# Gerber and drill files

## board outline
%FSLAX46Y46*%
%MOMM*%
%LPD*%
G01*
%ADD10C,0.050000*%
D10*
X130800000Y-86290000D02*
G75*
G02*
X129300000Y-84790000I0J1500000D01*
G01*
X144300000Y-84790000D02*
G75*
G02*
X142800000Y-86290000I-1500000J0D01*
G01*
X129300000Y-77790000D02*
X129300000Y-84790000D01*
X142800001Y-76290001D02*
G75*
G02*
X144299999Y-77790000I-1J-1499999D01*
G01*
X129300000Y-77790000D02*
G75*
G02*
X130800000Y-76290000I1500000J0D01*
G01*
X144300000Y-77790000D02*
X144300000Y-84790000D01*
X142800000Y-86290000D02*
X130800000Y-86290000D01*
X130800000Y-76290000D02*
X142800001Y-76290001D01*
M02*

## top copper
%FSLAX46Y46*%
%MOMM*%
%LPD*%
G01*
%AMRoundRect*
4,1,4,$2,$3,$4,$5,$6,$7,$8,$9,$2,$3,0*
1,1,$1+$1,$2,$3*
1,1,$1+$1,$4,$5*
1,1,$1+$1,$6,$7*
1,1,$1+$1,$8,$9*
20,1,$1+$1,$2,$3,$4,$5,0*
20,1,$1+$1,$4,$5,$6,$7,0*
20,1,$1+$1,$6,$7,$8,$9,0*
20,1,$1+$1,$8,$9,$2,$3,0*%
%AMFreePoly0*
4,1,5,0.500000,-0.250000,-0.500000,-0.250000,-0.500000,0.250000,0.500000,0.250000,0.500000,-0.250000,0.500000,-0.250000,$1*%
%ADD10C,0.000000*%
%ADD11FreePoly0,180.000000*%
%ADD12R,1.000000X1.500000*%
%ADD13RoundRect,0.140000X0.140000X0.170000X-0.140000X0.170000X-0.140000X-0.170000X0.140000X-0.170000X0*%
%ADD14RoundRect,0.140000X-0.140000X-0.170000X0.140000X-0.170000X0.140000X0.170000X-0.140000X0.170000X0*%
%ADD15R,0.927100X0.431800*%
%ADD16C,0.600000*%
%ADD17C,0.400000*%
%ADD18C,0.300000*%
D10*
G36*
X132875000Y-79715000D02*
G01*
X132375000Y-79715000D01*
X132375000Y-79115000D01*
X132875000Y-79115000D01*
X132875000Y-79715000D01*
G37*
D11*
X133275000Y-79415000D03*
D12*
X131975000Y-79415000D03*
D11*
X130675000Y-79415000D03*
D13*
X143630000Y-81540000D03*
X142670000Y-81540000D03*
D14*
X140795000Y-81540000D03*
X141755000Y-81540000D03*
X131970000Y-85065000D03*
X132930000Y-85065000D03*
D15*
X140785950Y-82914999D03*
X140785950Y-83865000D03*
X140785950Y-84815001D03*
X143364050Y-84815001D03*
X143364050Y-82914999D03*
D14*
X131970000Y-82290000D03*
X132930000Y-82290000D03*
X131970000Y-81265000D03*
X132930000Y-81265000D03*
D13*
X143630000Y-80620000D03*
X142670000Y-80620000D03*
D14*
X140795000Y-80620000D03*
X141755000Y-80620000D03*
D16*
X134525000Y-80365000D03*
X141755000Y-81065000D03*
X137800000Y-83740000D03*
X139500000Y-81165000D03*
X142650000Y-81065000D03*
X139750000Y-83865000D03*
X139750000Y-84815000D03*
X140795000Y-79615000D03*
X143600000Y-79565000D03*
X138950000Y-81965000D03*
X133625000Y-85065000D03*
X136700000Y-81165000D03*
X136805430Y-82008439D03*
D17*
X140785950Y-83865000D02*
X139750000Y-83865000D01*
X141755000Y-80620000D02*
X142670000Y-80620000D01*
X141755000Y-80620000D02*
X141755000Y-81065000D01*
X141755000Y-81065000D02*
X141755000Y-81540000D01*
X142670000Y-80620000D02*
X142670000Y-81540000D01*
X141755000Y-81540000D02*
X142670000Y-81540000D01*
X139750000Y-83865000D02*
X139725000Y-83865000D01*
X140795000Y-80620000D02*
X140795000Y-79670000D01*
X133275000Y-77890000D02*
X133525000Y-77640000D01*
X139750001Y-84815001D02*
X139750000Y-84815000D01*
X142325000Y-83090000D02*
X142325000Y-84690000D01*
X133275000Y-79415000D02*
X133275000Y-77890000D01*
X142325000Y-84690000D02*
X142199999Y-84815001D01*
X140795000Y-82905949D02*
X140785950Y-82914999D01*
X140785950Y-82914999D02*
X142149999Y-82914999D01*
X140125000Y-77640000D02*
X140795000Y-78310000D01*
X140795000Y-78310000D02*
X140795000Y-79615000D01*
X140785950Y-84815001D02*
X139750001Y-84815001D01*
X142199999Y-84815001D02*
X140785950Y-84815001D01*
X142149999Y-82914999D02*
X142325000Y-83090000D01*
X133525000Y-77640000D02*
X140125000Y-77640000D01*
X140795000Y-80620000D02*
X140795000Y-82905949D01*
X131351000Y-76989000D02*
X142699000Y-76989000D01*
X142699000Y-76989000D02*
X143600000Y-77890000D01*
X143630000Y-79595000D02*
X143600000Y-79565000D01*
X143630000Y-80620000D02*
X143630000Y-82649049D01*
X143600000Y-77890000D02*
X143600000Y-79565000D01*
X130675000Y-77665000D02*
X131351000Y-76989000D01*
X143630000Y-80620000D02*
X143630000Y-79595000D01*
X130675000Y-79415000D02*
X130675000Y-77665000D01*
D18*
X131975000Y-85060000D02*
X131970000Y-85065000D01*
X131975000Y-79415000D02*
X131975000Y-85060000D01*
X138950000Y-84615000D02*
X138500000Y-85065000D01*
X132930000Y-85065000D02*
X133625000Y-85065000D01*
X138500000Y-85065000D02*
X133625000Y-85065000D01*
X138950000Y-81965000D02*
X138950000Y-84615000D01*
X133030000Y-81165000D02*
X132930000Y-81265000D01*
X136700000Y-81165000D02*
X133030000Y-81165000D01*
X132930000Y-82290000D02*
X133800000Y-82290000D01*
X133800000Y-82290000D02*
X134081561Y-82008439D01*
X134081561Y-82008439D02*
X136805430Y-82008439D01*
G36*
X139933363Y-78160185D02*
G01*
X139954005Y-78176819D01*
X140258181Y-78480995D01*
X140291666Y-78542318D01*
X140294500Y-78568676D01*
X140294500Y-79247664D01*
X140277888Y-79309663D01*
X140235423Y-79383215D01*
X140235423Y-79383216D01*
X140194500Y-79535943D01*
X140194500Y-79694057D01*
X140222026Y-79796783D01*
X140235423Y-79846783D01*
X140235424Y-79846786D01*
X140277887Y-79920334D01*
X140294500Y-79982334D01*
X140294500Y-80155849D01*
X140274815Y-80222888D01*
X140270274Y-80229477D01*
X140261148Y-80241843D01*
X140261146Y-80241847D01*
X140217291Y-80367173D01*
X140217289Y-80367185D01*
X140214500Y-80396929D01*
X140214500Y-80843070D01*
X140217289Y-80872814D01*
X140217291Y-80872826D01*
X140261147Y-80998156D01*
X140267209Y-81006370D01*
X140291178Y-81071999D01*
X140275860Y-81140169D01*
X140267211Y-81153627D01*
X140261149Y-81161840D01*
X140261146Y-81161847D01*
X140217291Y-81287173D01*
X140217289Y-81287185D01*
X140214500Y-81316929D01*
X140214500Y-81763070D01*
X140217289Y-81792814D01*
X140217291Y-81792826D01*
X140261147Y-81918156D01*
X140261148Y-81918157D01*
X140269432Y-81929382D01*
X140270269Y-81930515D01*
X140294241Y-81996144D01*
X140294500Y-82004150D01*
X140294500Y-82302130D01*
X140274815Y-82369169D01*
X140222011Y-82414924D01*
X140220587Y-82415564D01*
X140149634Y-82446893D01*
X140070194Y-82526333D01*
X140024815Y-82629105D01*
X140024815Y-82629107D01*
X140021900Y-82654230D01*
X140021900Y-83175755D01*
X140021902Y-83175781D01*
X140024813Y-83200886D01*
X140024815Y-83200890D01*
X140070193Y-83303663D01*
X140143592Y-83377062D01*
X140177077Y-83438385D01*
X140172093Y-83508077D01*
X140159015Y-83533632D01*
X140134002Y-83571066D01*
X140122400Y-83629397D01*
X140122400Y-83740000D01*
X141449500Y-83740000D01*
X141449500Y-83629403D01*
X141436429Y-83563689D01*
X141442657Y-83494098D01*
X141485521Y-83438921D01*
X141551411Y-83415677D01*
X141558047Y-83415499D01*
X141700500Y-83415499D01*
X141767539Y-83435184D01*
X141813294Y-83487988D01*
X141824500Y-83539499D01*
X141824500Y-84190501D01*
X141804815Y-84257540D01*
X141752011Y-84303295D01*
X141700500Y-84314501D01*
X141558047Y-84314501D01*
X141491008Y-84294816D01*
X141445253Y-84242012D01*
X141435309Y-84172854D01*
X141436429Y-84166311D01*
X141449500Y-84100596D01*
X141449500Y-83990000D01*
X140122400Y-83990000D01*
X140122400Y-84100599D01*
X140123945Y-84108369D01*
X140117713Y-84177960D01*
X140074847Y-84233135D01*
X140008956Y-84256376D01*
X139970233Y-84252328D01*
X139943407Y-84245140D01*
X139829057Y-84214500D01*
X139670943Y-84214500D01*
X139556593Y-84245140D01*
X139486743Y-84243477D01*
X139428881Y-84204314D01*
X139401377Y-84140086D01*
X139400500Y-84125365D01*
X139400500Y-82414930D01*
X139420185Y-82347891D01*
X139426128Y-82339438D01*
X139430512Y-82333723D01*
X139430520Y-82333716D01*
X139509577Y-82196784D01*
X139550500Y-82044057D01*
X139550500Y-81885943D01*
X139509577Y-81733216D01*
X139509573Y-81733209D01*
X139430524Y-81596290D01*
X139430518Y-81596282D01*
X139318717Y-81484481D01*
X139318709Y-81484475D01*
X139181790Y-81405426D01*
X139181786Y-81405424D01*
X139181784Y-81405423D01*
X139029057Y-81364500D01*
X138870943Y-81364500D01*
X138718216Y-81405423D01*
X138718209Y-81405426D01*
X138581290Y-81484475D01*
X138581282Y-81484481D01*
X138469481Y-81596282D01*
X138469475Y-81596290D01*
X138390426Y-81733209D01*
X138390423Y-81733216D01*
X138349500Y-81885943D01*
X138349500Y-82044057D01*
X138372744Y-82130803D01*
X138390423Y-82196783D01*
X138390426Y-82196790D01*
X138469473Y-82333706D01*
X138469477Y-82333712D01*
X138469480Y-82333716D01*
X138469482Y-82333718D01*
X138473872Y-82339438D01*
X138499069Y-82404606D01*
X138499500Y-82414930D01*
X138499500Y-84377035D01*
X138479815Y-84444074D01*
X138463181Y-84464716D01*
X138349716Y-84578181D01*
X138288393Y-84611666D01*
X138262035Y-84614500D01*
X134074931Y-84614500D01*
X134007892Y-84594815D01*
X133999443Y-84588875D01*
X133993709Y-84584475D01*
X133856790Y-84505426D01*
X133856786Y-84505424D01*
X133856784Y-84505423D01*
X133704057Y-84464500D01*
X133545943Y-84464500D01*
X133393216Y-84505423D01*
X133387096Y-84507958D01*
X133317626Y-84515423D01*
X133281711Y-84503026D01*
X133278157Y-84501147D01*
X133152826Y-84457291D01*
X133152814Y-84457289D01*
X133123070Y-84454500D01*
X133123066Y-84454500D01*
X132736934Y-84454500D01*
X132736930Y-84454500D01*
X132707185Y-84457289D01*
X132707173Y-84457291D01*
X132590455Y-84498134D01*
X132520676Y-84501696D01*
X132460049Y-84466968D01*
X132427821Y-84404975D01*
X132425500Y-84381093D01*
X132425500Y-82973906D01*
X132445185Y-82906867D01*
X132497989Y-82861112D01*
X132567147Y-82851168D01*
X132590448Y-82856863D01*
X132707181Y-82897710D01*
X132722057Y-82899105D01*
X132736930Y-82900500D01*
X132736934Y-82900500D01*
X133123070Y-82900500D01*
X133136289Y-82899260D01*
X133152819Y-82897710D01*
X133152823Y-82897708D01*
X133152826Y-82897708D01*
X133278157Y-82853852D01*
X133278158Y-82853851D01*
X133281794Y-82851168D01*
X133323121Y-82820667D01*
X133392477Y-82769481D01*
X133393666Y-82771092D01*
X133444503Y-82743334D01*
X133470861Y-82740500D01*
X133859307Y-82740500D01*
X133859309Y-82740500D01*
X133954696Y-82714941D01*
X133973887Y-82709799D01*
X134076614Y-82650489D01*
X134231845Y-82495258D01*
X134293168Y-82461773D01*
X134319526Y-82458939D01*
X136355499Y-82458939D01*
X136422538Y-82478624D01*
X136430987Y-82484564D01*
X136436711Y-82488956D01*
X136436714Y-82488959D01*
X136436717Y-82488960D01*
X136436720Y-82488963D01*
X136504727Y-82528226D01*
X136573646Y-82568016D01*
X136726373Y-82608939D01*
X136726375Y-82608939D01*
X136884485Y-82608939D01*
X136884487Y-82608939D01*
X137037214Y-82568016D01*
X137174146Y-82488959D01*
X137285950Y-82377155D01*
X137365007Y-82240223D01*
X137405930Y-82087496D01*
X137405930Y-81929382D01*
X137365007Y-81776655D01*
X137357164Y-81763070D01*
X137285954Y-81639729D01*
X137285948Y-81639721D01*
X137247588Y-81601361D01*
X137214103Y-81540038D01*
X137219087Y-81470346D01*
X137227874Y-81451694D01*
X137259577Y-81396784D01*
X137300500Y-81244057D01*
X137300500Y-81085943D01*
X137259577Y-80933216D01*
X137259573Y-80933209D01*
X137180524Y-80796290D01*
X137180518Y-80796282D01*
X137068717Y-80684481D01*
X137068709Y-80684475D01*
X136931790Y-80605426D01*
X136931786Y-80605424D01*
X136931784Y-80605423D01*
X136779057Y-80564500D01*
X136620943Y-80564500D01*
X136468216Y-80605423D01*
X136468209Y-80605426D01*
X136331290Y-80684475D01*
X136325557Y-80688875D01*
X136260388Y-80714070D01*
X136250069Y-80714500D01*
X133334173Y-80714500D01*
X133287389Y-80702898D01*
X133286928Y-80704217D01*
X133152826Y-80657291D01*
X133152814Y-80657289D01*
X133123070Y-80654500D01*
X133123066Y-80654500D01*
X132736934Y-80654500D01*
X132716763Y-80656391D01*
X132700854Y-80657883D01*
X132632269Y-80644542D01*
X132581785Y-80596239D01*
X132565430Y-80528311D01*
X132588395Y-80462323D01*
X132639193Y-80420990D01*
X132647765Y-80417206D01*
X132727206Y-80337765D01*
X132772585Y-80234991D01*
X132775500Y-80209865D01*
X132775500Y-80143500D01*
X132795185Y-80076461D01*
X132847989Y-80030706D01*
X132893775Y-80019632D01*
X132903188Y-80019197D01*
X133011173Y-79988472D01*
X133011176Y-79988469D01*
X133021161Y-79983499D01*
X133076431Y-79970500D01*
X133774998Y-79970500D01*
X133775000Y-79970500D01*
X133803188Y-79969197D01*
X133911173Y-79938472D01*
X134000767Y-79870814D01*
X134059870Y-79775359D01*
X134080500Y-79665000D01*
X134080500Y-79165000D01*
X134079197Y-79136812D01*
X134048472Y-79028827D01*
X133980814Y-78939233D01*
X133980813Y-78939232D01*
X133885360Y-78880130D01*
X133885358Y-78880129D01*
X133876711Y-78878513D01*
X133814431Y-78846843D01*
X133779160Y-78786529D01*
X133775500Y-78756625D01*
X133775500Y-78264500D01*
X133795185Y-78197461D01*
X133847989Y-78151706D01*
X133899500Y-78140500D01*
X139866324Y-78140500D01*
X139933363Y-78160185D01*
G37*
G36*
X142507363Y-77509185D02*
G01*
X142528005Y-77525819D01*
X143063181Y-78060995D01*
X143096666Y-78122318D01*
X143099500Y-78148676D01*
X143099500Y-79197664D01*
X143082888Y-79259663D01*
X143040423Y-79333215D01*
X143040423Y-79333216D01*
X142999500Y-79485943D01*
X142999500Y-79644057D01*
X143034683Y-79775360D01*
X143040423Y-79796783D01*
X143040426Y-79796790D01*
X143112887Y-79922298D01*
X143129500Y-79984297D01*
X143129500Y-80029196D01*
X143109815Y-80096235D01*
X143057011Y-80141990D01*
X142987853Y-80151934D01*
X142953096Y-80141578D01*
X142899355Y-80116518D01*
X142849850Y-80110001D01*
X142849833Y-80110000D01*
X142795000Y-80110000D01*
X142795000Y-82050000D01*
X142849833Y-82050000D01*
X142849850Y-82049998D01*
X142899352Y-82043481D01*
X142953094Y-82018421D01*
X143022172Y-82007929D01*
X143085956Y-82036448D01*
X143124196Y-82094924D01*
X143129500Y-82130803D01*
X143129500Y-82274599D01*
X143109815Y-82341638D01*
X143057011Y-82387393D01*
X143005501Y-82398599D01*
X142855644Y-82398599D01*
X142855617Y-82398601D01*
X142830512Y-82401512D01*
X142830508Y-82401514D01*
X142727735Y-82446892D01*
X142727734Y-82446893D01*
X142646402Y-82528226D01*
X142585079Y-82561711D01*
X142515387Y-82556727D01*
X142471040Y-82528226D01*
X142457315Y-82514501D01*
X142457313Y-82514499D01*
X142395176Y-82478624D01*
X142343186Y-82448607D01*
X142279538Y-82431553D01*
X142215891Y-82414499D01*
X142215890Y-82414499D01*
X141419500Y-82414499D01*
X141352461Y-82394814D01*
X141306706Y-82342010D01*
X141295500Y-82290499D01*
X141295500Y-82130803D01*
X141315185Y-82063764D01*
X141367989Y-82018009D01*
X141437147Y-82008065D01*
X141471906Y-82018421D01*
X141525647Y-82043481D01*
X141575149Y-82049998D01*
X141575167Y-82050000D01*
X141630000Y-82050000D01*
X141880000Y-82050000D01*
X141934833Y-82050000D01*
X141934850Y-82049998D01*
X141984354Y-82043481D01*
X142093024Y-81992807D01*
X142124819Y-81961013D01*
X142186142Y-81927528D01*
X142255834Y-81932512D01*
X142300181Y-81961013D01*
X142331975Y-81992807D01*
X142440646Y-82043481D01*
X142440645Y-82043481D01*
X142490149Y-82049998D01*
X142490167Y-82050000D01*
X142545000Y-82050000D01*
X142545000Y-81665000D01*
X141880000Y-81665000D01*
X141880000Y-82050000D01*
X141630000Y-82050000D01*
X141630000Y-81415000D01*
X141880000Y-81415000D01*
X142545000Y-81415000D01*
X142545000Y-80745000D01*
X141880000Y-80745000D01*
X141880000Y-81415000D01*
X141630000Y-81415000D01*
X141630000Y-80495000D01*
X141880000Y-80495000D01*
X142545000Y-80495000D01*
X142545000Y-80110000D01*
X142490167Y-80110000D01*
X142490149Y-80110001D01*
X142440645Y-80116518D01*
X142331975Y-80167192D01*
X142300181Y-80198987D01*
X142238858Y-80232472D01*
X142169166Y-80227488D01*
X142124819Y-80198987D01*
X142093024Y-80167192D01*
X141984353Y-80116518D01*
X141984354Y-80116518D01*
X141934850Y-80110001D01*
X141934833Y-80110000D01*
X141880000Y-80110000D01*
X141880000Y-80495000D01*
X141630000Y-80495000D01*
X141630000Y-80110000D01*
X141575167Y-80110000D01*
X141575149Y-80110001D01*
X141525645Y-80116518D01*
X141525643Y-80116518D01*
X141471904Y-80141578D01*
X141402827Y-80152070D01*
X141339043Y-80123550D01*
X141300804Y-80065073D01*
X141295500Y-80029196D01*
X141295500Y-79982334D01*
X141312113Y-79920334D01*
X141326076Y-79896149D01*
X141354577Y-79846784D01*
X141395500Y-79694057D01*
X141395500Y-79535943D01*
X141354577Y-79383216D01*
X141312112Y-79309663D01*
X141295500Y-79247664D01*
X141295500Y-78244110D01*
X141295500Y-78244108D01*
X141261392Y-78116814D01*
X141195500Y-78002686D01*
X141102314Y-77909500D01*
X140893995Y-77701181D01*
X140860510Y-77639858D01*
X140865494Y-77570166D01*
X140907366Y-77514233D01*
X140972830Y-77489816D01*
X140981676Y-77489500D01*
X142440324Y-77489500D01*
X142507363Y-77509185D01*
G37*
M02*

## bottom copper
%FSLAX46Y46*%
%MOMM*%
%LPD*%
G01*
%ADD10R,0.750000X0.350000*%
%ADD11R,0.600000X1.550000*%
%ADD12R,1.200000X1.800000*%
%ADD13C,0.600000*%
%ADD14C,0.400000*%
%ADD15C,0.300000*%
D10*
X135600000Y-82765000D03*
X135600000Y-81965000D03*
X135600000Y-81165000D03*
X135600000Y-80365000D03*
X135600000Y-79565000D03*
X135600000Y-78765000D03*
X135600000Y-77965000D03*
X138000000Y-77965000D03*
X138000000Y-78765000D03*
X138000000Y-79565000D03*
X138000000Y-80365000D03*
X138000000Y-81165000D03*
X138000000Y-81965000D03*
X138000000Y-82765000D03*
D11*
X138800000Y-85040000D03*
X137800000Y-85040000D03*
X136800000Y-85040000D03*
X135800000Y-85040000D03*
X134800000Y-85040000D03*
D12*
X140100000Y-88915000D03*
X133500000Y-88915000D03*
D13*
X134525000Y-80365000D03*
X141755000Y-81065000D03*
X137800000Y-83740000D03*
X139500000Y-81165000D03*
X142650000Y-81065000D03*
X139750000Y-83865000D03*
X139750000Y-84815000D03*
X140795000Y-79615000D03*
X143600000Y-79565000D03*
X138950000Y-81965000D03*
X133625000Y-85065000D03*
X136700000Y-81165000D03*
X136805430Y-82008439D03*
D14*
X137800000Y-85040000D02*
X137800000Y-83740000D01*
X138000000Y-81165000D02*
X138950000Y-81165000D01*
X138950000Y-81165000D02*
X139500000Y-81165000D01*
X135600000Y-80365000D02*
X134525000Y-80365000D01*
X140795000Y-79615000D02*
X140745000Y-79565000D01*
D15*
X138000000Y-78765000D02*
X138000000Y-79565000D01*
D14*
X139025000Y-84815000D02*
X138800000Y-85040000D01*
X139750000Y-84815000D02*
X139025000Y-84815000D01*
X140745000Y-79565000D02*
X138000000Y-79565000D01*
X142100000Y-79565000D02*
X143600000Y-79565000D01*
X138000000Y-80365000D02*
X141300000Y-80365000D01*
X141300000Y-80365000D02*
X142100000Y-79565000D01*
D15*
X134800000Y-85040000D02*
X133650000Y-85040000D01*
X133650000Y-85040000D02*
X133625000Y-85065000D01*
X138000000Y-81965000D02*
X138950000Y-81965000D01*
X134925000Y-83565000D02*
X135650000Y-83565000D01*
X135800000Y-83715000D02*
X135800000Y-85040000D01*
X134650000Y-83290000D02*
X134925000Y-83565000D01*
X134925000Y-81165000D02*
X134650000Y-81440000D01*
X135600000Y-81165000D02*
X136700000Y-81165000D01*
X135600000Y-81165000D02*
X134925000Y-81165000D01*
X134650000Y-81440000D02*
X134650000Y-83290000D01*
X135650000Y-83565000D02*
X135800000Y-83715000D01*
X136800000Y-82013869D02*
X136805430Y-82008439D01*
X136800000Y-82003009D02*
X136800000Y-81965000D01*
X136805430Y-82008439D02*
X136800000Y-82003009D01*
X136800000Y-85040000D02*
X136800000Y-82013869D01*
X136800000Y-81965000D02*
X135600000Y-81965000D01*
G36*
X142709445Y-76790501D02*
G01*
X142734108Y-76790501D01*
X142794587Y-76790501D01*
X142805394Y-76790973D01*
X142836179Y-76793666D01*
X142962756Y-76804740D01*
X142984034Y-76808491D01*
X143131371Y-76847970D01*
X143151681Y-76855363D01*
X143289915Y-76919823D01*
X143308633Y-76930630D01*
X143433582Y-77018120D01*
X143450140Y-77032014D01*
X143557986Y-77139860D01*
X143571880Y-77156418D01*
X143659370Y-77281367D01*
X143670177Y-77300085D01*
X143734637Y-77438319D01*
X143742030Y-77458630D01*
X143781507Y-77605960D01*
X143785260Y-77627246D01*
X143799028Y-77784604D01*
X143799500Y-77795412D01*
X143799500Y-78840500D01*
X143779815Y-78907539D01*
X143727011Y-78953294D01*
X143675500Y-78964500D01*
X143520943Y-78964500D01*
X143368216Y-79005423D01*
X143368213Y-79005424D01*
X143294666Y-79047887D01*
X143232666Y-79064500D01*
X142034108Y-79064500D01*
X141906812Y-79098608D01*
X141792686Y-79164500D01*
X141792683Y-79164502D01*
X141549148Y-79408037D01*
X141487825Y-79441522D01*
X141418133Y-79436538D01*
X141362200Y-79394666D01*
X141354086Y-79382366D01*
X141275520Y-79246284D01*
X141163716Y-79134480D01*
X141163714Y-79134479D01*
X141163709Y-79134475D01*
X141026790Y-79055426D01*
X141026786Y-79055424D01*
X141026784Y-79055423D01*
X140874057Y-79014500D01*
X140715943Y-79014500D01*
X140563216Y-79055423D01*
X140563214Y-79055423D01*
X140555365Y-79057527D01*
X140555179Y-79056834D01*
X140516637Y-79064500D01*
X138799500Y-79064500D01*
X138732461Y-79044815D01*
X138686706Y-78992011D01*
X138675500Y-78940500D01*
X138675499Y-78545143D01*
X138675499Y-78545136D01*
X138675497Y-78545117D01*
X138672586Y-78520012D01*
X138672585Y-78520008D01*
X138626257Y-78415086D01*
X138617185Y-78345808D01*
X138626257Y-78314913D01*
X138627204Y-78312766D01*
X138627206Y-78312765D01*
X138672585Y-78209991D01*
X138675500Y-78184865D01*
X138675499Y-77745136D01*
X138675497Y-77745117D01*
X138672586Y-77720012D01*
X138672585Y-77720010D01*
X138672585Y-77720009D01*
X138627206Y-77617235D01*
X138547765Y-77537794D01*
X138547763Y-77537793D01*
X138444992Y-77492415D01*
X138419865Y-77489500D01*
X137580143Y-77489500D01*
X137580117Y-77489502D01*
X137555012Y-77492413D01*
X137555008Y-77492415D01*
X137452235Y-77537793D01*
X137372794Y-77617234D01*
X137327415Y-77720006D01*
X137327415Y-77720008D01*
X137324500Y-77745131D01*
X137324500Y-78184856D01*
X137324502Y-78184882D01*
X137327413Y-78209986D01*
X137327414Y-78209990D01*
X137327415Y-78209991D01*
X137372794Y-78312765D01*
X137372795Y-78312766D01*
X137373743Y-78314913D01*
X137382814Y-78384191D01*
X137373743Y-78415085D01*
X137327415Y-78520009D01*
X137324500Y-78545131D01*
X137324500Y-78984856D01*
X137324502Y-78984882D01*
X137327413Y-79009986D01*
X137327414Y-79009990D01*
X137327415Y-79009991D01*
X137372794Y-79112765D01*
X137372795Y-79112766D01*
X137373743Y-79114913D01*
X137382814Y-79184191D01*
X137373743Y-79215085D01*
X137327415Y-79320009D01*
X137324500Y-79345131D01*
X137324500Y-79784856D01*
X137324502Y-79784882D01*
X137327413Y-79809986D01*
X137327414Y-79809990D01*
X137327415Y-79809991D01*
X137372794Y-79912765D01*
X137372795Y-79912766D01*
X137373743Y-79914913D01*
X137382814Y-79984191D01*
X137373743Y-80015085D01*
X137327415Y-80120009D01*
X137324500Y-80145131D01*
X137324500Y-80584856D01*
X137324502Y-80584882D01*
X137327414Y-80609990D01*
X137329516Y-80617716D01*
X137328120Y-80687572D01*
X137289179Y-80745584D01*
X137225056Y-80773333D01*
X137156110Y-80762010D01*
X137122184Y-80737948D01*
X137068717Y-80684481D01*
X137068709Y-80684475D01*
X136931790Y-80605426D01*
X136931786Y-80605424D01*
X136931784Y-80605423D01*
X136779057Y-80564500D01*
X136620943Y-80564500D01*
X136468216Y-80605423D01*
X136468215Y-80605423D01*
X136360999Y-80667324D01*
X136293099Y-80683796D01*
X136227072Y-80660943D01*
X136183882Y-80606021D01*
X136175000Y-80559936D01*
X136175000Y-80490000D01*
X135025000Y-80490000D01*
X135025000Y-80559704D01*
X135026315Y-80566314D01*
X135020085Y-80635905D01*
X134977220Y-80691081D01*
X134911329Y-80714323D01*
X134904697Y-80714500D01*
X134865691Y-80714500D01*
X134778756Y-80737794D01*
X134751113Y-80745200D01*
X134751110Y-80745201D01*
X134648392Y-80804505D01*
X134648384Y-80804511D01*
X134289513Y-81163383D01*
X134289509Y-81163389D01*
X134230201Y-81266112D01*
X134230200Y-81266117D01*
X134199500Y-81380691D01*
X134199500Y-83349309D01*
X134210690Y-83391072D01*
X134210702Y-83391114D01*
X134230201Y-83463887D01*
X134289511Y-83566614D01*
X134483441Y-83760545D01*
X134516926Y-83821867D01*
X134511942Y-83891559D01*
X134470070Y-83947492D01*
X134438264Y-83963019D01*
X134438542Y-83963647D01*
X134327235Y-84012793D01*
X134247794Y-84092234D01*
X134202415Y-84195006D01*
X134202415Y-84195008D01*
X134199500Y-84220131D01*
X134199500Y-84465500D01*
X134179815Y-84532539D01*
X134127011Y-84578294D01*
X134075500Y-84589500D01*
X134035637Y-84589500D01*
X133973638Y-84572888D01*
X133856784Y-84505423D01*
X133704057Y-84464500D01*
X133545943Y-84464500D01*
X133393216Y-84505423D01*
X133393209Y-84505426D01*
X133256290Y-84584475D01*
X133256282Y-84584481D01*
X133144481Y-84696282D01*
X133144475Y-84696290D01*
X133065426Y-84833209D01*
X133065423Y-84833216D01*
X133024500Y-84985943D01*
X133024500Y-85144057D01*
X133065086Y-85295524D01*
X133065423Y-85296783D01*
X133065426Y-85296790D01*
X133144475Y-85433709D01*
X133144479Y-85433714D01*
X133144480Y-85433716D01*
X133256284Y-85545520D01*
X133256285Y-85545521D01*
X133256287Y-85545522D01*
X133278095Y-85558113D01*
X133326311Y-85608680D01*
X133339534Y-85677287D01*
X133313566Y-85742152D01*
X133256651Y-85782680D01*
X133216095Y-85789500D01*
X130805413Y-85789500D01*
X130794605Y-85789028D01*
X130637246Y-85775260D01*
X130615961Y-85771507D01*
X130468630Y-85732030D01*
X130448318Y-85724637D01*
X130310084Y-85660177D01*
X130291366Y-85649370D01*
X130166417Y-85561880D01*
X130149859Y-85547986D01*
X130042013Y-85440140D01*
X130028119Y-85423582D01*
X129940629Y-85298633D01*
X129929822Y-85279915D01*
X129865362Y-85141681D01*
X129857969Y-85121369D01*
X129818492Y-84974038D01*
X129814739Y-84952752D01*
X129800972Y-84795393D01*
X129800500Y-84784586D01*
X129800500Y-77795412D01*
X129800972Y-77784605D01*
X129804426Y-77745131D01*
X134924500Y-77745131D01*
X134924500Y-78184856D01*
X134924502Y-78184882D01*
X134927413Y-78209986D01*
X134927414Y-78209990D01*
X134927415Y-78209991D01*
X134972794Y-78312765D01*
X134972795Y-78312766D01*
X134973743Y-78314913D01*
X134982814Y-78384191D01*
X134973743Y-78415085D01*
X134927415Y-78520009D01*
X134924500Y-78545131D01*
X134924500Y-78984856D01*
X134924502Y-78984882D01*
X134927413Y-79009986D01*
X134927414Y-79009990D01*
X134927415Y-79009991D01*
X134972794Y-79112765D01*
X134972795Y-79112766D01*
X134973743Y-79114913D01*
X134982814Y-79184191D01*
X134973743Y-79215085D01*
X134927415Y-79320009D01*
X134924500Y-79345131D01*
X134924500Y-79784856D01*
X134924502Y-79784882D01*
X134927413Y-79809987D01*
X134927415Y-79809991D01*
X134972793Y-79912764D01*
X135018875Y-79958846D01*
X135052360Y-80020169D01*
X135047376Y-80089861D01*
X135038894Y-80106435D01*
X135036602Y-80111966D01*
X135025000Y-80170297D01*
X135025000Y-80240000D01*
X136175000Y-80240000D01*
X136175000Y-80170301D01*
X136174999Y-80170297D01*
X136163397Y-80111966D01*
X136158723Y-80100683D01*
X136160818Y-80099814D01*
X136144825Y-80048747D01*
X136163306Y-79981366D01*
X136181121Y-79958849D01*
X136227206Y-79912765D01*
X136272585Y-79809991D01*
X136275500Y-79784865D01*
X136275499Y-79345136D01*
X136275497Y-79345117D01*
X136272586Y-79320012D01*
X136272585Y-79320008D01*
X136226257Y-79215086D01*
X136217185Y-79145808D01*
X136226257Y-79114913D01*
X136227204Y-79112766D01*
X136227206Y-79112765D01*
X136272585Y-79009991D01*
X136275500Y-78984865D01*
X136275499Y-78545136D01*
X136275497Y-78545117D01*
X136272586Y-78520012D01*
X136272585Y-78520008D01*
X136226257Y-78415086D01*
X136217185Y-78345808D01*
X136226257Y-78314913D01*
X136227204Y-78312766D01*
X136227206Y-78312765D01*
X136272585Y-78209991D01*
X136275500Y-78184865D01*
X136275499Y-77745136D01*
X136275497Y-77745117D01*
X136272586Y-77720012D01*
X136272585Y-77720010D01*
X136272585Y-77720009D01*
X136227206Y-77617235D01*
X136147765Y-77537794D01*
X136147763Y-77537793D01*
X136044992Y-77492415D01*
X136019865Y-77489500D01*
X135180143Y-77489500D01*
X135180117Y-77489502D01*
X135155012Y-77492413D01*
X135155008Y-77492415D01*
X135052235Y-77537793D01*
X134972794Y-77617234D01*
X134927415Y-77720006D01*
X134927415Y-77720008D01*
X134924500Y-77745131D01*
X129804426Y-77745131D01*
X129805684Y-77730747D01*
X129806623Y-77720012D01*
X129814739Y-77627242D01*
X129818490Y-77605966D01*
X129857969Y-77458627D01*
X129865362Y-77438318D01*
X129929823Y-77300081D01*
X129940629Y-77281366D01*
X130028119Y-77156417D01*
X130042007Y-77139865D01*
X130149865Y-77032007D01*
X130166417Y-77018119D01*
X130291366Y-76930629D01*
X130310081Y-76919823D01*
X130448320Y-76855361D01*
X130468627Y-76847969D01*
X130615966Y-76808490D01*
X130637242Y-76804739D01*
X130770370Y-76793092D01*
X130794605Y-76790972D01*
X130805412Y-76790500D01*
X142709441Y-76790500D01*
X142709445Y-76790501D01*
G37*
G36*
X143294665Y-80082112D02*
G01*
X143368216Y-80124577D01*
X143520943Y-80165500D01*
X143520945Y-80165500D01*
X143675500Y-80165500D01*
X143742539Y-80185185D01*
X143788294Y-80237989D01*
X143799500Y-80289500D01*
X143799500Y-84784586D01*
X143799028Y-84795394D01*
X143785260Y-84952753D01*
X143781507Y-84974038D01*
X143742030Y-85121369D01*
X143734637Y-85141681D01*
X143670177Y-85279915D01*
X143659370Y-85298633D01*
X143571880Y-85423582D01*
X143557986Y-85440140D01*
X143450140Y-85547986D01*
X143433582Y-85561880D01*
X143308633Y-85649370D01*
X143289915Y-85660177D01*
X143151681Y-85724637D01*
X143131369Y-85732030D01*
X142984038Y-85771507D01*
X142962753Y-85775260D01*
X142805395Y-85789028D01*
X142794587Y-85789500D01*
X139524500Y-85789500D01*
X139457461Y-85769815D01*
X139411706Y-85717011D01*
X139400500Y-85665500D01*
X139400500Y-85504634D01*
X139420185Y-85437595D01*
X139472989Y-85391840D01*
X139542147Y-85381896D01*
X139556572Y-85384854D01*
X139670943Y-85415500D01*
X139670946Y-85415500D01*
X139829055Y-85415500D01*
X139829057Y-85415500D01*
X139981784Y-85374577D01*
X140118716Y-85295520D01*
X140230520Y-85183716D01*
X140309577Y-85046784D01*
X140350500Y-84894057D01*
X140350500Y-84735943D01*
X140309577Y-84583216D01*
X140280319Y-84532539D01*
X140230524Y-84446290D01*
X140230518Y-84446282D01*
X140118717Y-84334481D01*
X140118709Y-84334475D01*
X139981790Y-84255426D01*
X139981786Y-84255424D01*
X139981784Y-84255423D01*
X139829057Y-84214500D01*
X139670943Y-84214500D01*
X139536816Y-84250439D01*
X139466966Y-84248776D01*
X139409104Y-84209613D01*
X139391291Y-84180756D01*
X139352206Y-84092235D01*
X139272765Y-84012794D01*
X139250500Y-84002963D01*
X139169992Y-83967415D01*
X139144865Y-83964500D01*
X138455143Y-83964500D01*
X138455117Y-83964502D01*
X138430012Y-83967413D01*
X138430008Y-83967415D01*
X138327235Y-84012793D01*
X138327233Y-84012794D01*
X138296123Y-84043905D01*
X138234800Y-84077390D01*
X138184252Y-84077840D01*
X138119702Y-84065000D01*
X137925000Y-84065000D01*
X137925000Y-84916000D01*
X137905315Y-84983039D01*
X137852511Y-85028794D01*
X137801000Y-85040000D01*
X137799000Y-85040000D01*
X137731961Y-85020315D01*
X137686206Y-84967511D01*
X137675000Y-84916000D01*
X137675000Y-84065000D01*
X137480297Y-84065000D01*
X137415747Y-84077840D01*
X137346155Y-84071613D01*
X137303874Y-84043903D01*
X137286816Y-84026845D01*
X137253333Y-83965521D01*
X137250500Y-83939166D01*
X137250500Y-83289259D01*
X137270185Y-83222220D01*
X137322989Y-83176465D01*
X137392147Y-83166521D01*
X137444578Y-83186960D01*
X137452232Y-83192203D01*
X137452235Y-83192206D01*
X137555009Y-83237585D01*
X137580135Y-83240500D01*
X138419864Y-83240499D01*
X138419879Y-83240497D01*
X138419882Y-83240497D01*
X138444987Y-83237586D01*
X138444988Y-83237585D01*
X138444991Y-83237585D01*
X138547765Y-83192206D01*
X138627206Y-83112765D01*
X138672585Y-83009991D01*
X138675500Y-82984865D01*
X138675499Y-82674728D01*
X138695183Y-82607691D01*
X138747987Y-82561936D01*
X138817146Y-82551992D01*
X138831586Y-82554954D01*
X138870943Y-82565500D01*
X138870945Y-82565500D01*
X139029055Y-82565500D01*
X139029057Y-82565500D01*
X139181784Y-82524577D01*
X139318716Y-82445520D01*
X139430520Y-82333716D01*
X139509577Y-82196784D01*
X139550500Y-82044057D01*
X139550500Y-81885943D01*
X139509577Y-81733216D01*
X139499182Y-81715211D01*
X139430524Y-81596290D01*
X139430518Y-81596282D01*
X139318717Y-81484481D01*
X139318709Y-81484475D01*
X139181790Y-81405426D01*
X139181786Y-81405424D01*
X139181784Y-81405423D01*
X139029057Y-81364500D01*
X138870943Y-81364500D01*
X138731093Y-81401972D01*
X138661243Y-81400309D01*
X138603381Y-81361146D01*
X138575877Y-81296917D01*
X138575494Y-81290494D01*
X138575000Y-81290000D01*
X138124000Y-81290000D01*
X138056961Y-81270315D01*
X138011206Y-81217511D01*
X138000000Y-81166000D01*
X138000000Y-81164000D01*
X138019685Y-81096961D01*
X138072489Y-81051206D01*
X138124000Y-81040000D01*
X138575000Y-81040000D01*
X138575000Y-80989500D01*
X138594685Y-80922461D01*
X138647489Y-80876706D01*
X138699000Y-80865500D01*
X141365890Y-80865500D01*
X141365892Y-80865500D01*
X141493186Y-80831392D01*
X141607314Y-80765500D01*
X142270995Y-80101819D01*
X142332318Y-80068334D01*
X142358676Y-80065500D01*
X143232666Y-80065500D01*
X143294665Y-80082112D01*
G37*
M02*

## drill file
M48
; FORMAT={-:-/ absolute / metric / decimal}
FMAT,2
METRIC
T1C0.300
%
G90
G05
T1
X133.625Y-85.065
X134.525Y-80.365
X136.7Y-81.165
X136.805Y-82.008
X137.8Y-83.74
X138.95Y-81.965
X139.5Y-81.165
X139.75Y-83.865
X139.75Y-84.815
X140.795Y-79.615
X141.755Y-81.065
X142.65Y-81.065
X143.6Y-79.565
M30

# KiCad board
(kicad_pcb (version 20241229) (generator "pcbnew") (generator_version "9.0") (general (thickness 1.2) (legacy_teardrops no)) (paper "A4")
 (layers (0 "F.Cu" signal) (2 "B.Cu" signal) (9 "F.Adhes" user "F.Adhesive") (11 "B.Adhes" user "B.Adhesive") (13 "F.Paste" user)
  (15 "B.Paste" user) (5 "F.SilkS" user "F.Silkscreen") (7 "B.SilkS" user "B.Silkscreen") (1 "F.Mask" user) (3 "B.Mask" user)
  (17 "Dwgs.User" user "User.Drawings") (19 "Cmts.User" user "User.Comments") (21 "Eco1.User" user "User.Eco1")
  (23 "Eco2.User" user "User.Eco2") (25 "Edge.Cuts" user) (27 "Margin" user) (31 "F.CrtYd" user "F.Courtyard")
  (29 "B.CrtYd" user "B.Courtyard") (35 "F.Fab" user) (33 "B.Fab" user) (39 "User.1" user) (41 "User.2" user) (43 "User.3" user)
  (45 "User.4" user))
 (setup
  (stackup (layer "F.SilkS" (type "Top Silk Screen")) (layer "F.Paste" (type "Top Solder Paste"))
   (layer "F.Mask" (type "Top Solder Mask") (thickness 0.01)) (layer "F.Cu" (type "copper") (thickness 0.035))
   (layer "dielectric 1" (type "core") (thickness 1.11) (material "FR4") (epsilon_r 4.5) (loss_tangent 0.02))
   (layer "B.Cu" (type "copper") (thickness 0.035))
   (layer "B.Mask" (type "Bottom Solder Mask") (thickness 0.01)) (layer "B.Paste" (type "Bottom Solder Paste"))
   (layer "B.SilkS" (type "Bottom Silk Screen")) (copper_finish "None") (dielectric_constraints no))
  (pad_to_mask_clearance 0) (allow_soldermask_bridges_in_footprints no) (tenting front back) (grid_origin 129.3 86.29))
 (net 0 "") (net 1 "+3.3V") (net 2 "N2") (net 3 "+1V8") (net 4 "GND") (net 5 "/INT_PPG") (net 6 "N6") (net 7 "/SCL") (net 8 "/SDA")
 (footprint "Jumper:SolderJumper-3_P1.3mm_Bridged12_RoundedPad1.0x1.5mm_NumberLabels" (layer "F.Cu") (at 131.975 79.415 180)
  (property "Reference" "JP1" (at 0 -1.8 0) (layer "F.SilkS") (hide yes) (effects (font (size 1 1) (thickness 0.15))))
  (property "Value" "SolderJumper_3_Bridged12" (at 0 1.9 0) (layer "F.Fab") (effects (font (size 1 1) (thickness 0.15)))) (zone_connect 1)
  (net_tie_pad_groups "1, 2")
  (fp_poly (pts (xy -0.9 -0.3) (xy -0.4 -0.3) (xy -0.4 0.3) (xy -0.9 0.3)) (stroke (width 0) (type solid)) (fill yes) (layer "F.Cu"))
  (pad "1" smd custom (at -1.3 0 180) (size 1 0.5) (layers "F.Cu" "F.Mask") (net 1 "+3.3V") (zone_connect 2) (thermal_bridge_angle 45)
   (options (clearance outline) (anchor rect)) (primitives))
  (pad "2" smd rect (at 0 0 180) (size 1 1.5) (layers "F.Cu" "F.Mask") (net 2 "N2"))
  (pad "3" smd custom (at 1.3 0 180) (size 1 0.5) (layers "F.Cu" "F.Mask") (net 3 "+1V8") (zone_connect 2) (thermal_bridge_angle 45)
   (options (clearance outline) (anchor rect)) (primitives)))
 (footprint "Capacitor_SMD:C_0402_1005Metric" (layer "F.Cu") (at 143.15 81.54 180)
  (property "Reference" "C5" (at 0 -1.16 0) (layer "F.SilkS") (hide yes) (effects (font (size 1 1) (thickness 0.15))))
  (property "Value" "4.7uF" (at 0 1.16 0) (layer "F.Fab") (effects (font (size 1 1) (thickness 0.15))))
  (pad "1" smd roundrect (at -0.48 0 180) (size 0.56 0.62) (layers "F.Cu" "F.Mask" "F.Paste") (roundrect_rratio 0.25) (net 3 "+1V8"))
  (pad "2" smd roundrect (at 0.48 0 180) (size 0.56 0.62) (layers "F.Cu" "F.Mask" "F.Paste") (roundrect_rratio 0.25) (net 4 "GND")))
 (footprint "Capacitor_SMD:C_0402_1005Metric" (layer "F.Cu") (at 141.275 81.54)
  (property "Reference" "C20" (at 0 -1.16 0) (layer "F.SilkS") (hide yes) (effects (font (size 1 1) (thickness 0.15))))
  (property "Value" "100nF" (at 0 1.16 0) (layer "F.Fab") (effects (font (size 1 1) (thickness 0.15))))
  (pad "1" smd roundrect (at -0.48 0) (size 0.56 0.62) (layers "F.Cu" "F.Mask" "F.Paste") (roundrect_rratio 0.25) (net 1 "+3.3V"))
  (pad "2" smd roundrect (at 0.48 0) (size 0.56 0.62) (layers "F.Cu" "F.Mask" "F.Paste") (roundrect_rratio 0.25) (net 4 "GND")))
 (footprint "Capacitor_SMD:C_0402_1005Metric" (layer "F.Cu") (at 132.45 85.065)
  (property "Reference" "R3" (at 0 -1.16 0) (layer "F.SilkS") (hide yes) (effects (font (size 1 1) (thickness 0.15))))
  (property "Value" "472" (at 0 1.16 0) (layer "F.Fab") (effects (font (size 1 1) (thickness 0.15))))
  (pad "1" smd roundrect (at -0.48 0) (size 0.56 0.62) (layers "F.Cu" "F.Mask" "F.Paste") (roundrect_rratio 0.25) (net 2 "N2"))
  (pad "2" smd roundrect (at 0.48 0) (size 0.56 0.62) (layers "F.Cu" "F.Mask" "F.Paste") (roundrect_rratio 0.25) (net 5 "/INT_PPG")))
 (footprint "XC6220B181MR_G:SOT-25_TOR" (layer "F.Cu") (at 142.075 83.865)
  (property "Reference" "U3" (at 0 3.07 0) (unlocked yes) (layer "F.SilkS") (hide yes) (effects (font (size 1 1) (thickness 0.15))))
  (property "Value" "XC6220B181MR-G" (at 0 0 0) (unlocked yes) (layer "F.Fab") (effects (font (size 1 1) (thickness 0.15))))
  (pad "1" smd rect (at -1.28905 -0.950001) (size 0.9271 0.4318) (layers "F.Cu" "F.Mask" "F.Paste") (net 1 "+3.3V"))
  (pad "2" smd rect (at -1.28905 0) (size 0.9271 0.4318) (layers "F.Cu" "F.Mask" "F.Paste") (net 4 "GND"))
  (pad "3" smd rect (at -1.28905 0.950001) (size 0.9271 0.4318) (layers "F.Cu" "F.Mask" "F.Paste") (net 1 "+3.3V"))
  (pad "4" smd rect (at 1.28905 0.950001) (size 0.9271 0.4318) (layers "F.Cu" "F.Mask" "F.Paste") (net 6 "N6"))
  (pad "5" smd rect (at 1.28905 -0.950001) (size 0.9271 0.4318) (layers "F.Cu" "F.Mask" "F.Paste") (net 3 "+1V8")))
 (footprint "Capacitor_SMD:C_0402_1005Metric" (layer "F.Cu") (at 132.45 82.29)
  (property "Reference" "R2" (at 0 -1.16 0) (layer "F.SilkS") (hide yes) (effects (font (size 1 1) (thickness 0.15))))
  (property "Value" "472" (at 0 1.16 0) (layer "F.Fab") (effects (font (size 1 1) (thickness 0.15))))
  (pad "1" smd roundrect (at -0.48 0) (size 0.56 0.62) (layers "F.Cu" "F.Mask" "F.Paste") (roundrect_rratio 0.25) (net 2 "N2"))
  (pad "2" smd roundrect (at 0.48 0) (size 0.56 0.62) (layers "F.Cu" "F.Mask" "F.Paste") (roundrect_rratio 0.25) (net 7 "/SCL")))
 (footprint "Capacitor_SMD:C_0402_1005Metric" (layer "F.Cu") (at 132.45 81.265)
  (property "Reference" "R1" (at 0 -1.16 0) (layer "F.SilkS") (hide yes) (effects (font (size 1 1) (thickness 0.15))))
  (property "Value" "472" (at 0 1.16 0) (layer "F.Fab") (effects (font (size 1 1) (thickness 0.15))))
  (pad "1" smd roundrect (at -0.48 0) (size 0.56 0.62) (layers "F.Cu" "F.Mask" "F.Paste") (roundrect_rratio 0.25) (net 2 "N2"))
  (pad "2" smd roundrect (at 0.48 0) (size 0.56 0.62) (layers "F.Cu" "F.Mask" "F.Paste") (roundrect_rratio 0.25) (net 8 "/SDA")))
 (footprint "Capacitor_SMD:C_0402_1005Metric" (layer "F.Cu") (at 143.15 80.62 180)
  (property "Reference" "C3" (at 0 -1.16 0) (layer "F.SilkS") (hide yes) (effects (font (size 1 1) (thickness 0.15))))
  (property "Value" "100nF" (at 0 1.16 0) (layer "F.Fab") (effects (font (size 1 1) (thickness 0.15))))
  (pad "1" smd roundrect (at -0.48 0 180) (size 0.56 0.62) (layers "F.Cu" "F.Mask" "F.Paste") (roundrect_rratio 0.25) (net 3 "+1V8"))
  (pad "2" smd roundrect (at 0.48 0 180) (size 0.56 0.62) (layers "F.Cu" "F.Mask" "F.Paste") (roundrect_rratio 0.25) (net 4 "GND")))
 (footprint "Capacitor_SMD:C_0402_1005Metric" (layer "F.Cu") (at 141.275 80.62)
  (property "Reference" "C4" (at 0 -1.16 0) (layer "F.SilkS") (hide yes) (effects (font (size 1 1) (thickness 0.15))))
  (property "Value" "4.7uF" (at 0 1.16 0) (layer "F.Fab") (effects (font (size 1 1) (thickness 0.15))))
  (pad "1" smd roundrect (at -0.48 0) (size 0.56 0.62) (layers "F.Cu" "F.Mask" "F.Paste") (roundrect_rratio 0.25) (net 1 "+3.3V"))
  (pad "2" smd roundrect (at 0.48 0) (size 0.56 0.62) (layers "F.Cu" "F.Mask" "F.Paste") (roundrect_rratio 0.25) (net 4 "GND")))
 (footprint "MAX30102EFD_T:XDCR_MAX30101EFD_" (layer "B.Cu") (at 136.8 80.365)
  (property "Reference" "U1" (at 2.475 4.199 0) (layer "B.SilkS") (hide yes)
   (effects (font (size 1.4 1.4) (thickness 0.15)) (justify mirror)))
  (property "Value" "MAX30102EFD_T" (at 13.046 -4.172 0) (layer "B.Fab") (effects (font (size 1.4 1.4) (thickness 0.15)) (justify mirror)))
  (pad "1" smd rect (at -1.2 2.4) (size 0.75 0.35) (layers "B.Cu" "B.Mask" "B.Paste") (solder_mask_margin 0.102))
  (pad "2" smd rect (at -1.2 1.6) (size 0.75 0.35) (layers "B.Cu" "B.Mask" "B.Paste") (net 7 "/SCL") (solder_mask_margin 0.102))
  (pad "3" smd rect (at -1.2 0.8) (size 0.75 0.35) (layers "B.Cu" "B.Mask" "B.Paste") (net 8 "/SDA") (solder_mask_margin 0.102))
  (pad "4" smd rect (at -1.2 0) (size 0.75 0.35) (layers "B.Cu" "B.Mask" "B.Paste") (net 4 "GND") (solder_mask_margin 0.102))
  (pad "5" smd rect (at -1.2 -0.8) (size 0.75 0.35) (layers "B.Cu" "B.Mask" "B.Paste") (solder_mask_margin 0.102))
  (pad "6" smd rect (at -1.2 -1.6) (size 0.75 0.35) (layers "B.Cu" "B.Mask" "B.Paste") (solder_mask_margin 0.102))
  (pad "7" smd rect (at -1.2 -2.4) (size 0.75 0.35) (layers "B.Cu" "B.Mask" "B.Paste") (solder_mask_margin 0.102))
  (pad "8" smd rect (at 1.2 -2.4 180) (size 0.75 0.35) (layers "B.Cu" "B.Mask" "B.Paste") (solder_mask_margin 0.102))
  (pad "9" smd rect (at 1.2 -1.6 180) (size 0.75 0.35) (layers "B.Cu" "B.Mask" "B.Paste") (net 1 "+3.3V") (solder_mask_margin 0.102))
  (pad "10" smd rect (at 1.2 -0.8 180) (size 0.75 0.35) (layers "B.Cu" "B.Mask" "B.Paste") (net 1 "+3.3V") (solder_mask_margin 0.102))
  (pad "11" smd rect (at 1.2 0 180) (size 0.75 0.35) (layers "B.Cu" "B.Mask" "B.Paste") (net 3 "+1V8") (solder_mask_margin 0.102))
  (pad "12" smd rect (at 1.2 0.8 180) (size 0.75 0.35) (layers "B.Cu" "B.Mask" "B.Paste") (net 4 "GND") (solder_mask_margin 0.102))
  (pad "13" smd rect (at 1.2 1.6 180) (size 0.75 0.35) (layers "B.Cu" "B.Mask" "B.Paste") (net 5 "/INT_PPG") (solder_mask_margin 0.102))
  (pad "14" smd rect (at 1.2 2.4 180) (size 0.75 0.35) (layers "B.Cu" "B.Mask" "B.Paste") (solder_mask_margin 0.102)))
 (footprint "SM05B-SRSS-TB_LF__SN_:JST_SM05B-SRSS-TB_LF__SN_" (layer "B.Cu") (at 136.8 88.915 180)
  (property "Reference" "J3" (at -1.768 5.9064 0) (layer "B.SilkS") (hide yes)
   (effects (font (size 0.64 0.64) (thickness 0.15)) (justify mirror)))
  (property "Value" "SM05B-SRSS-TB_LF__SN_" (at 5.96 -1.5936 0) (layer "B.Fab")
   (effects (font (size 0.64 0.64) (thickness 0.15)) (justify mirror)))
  (pad "1" smd rect (at -2 3.875 180) (size 0.6 1.55) (layers "B.Cu" "B.Mask" "B.Paste") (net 1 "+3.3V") (solder_mask_margin 0.102))
  (pad "2" smd rect (at -1 3.875 180) (size 0.6 1.55) (layers "B.Cu" "B.Mask" "B.Paste") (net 4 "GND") (solder_mask_margin 0.102))
  (pad "3" smd rect (at 0 3.875 180) (size 0.6 1.55) (layers "B.Cu" "B.Mask" "B.Paste") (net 7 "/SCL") (solder_mask_margin 0.102))
  (pad "4" smd rect (at 1 3.875 180) (size 0.6 1.55) (layers "B.Cu" "B.Mask" "B.Paste") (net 8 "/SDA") (solder_mask_margin 0.102))
  (pad "5" smd rect (at 2 3.875 180) (size 0.6 1.55) (layers "B.Cu" "B.Mask" "B.Paste") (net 5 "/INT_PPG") (solder_mask_margin 0.102))
  (pad "S1" smd rect (at -3.3 0 180) (size 1.2 1.8) (layers "B.Cu" "B.Mask" "B.Paste") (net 4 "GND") (solder_mask_margin 0.102))
  (pad "S2" smd rect (at 3.3 0 180) (size 1.2 1.8) (layers "B.Cu" "B.Mask" "B.Paste") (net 4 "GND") (solder_mask_margin 0.102)))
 (gr_arc (start 130.8 86.29) (mid 129.73934 85.85066) (end 129.3 84.79) (stroke (width 0.05) (type default)) (layer "Edge.Cuts"))
 (gr_arc (start 144.3 84.79) (mid 143.86066 85.85066) (end 142.8 86.29) (stroke (width 0.05) (type default)) (layer "Edge.Cuts"))
 (gr_line (start 129.3 77.79) (end 129.3 84.79) (stroke (width 0.05) (type default)) (layer "Edge.Cuts"))
 (gr_arc (start 142.800001 76.290001) (mid 143.86066 76.729341) (end 144.3 77.79) (stroke (width 0.05) (type default)) (layer "Edge.Cuts"))
 (gr_arc (start 129.3 77.79) (mid 129.73934 76.72934) (end 130.8 76.29) (stroke (width 0.05) (type default)) (layer "Edge.Cuts"))
 (gr_line (start 144.3 77.79) (end 144.3 84.79) (stroke (width 0.05) (type default)) (layer "Edge.Cuts"))
 (gr_line (start 142.8 86.29) (end 130.8 86.29) (stroke (width 0.05) (type default)) (layer "Edge.Cuts"))
 (gr_line (start 130.8 76.29) (end 142.800001 76.290001) (stroke (width 0.05) (type default)) (layer "Edge.Cuts"))
 (segment (start 140.78595 83.865) (end 139.75 83.865) (width 0.4) (layer "F.Cu") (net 4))
 (segment (start 141.755 80.62) (end 142.67 80.62) (width 0.4) (layer "F.Cu") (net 4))
 (segment (start 141.755 80.62) (end 141.755 81.065) (width 0.4) (layer "F.Cu") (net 4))
 (segment (start 141.755 81.065) (end 141.755 81.54) (width 0.4) (layer "F.Cu") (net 4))
 (segment (start 142.67 80.62) (end 142.67 81.54) (width 0.4) (layer "F.Cu") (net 4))
 (segment (start 141.755 81.54) (end 142.67 81.54) (width 0.4) (layer "F.Cu") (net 4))
 (segment (start 139.75 83.865) (end 139.725 83.865) (width 0.4) (layer "F.Cu") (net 4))
 (via (at 134.525 80.365) (size 0.6) (drill 0.3) (layers "F.Cu" "B.Cu") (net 4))
 (via (at 141.755 81.065) (size 0.6) (drill 0.3) (layers "F.Cu" "B.Cu") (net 4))
 (via (at 137.8 83.74) (size 0.6) (drill 0.3) (layers "F.Cu" "B.Cu") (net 4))
 (via (at 139.5 81.165) (size 0.6) (drill 0.3) (layers "F.Cu" "B.Cu") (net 4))
 (via (at 142.65 81.065) (size 0.6) (drill 0.3) (layers "F.Cu" "B.Cu") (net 4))
 (via (at 139.75 83.865) (size 0.6) (drill 0.3) (layers "F.Cu" "B.Cu") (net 4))
 (segment (start 137.8 85.04) (end 137.8 83.74) (width 0.4) (layer "B.Cu") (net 4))
 (segment (start 138 81.165) (end 138.95 81.165) (width 0.4) (layer "B.Cu") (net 4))
 (segment (start 138.95 81.165) (end 139.5 81.165) (width 0.4) (layer "B.Cu") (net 4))
 (segment (start 135.6 80.365) (end 134.525 80.365) (width 0.4) (layer "B.Cu") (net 4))
 (segment (start 140.795 80.62) (end 140.795 79.67) (width 0.4) (layer "F.Cu") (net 1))
 (segment (start 133.275 77.89) (end 133.525 77.64) (width 0.4) (layer "F.Cu") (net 1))
 (segment (start 139.750001 84.815001) (end 139.75 84.815) (width 0.4) (layer "F.Cu") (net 1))
 (segment (start 142.325 83.09) (end 142.325 84.69) (width 0.4) (layer "F.Cu") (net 1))
 (segment (start 133.275 79.415) (end 133.275 77.89) (width 0.4) (layer "F.Cu") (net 1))
 (segment (start 142.325 84.69) (end 142.199999 84.815001) (width 0.4) (layer "F.Cu") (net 1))
 (segment (start 140.795 82.905949) (end 140.78595 82.914999) (width 0.4) (layer "F.Cu") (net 1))
 (segment (start 140.78595 82.914999) (end 142.149999 82.914999) (width 0.4) (layer "F.Cu") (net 1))
 (segment (start 140.125 77.64) (end 140.795 78.31) (width 0.4) (layer "F.Cu") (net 1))
 (segment (start 140.795 78.31) (end 140.795 79.615) (width 0.4) (layer "F.Cu") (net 1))
 (segment (start 140.78595 84.815001) (end 139.750001 84.815001) (width 0.4) (layer "F.Cu") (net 1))
 (segment (start 142.199999 84.815001) (end 140.78595 84.815001) (width 0.4) (layer "F.Cu") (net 1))
 (segment (start 142.149999 82.914999) (end 142.325 83.09) (width 0.4) (layer "F.Cu") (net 1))
 (segment (start 133.525 77.64) (end 140.125 77.64) (width 0.4) (layer "F.Cu") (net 1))
 (segment (start 140.795 80.62) (end 140.795 82.905949) (width 0.4) (layer "F.Cu") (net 1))
 (via (at 139.75 84.815) (size 0.6) (drill 0.3) (layers "F.Cu" "B.Cu") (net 1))
 (via (at 140.795 79.615) (size 0.6) (drill 0.3) (layers "F.Cu" "B.Cu") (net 1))
 (segment (start 140.795 79.615) (end 140.745 79.565) (width 0.4) (layer "B.Cu") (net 1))
 (segment (start 138 78.765) (end 138 79.565) (width 0.3) (layer "B.Cu") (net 1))
 (segment (start 139.025 84.815) (end 138.8 85.04) (width 0.4) (layer "B.Cu") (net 1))
 (segment (start 139.75 84.815) (end 139.025 84.815) (width 0.4) (layer "B.Cu") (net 1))
 (segment (start 140.745 79.565) (end 138 79.565) (width 0.4) (layer "B.Cu") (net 1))
 (segment (start 131.351 76.989) (end 142.699 76.989) (width 0.4) (layer "F.Cu") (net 3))
 (segment (start 142.699 76.989) (end 143.6 77.89) (width 0.4) (layer "F.Cu") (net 3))
 (segment (start 143.63 79.595) (end 143.6 79.565) (width 0.4) (layer "F.Cu") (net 3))
 (segment (start 143.63 80.62) (end 143.63 82.649049) (width 0.4) (layer "F.Cu") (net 3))
 (segment (start 143.6 77.89) (end 143.6 79.565) (width 0.4) (layer "F.Cu") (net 3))
 (segment (start 130.675 77.665) (end 131.351 76.989) (width 0.4) (layer "F.Cu") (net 3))
 (segment (start 143.63 80.62) (end 143.63 79.595) (width 0.4) (layer "F.Cu") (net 3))
 (segment (start 130.675 79.415) (end 130.675 77.665) (width 0.4) (layer "F.Cu") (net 3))
 (via (at 143.6 79.565) (size 0.6) (drill 0.3) (layers "F.Cu" "B.Cu") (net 3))
 (segment (start 142.1 79.565) (end 143.6 79.565) (width 0.4) (layer "B.Cu") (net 3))
 (segment (start 138 80.365) (end 141.3 80.365) (width 0.4) (layer "B.Cu") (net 3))
 (segment (start 141.3 80.365) (end 142.1 79.565) (width 0.4) (layer "B.Cu") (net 3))
 (segment (start 131.975 85.06) (end 131.97 85.065) (width 0.3) (layer "F.Cu") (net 2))
 (segment (start 131.975 79.415) (end 131.975 85.06) (width 0.3) (layer "F.Cu") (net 2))
 (segment (start 138.95 84.615) (end 138.5 85.065) (width 0.3) (layer "F.Cu") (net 5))
 (segment (start 132.93 85.065) (end 133.625 85.065) (width 0.3) (layer "F.Cu") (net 5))
 (segment (start 138.5 85.065) (end 133.625 85.065) (width 0.3) (layer "F.Cu") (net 5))
 (segment (start 138.95 81.965) (end 138.95 84.615) (width 0.3) (layer "F.Cu") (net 5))
 (via (at 138.95 81.965) (size 0.6) (drill 0.3) (layers "F.Cu" "B.Cu") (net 5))
 (via (at 133.625 85.065) (size 0.6) (drill 0.3) (layers "F.Cu" "B.Cu") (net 5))
 (segment (start 134.8 85.04) (end 133.65 85.04) (width 0.3) (layer "B.Cu") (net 5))
 (segment (start 133.65 85.04) (end 133.625 85.065) (width 0.3) (layer "B.Cu") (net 5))
 (segment (start 138 81.965) (end 138.95 81.965) (width 0.3) (layer "B.Cu") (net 5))
 (segment (start 133.03 81.165) (end 132.93 81.265) (width 0.3) (layer "F.Cu") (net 8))
 (segment (start 136.7 81.165) (end 133.03 81.165) (width 0.3) (layer "F.Cu") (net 8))
 (via (at 136.7 81.165) (size 0.6) (drill 0.3) (layers "F.Cu" "B.Cu") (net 8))
 (segment (start 134.925 83.565) (end 135.65 83.565) (width 0.3) (layer "B.Cu") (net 8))
 (segment (start 135.8 83.715) (end 135.8 85.04) (width 0.3) (layer "B.Cu") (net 8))
 (segment (start 134.65 83.29) (end 134.925 83.565) (width 0.3) (layer "B.Cu") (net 8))
 (segment (start 134.925 81.165) (end 134.65 81.44) (width 0.3) (layer "B.Cu") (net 8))
 (segment (start 135.6 81.165) (end 136.7 81.165) (width 0.3) (layer "B.Cu") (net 8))
 (segment (start 135.6 81.165) (end 134.925 81.165) (width 0.3) (layer "B.Cu") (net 8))
 (segment (start 134.65 81.44) (end 134.65 83.29) (width 0.3) (layer "B.Cu") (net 8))
 (segment (start 135.65 83.565) (end 135.8 83.715) (width 0.3) (layer "B.Cu") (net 8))
 (segment (start 132.93 82.29) (end 133.8 82.29) (width 0.3) (layer "F.Cu") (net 7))
 (segment (start 133.8 82.29) (end 134.081561 82.008439) (width 0.3) (layer "F.Cu") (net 7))
 (segment (start 134.081561 82.008439) (end 136.80543 82.008439) (width 0.3) (layer "F.Cu") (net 7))
 (via (at 136.80543 82.008439) (size 0.6) (drill 0.3) (layers "F.Cu" "B.Cu") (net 7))
 (segment (start 136.8 82.013869) (end 136.80543 82.008439) (width 0.3) (layer "B.Cu") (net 7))
 (segment (start 136.8 82.003009) (end 136.8 81.965) (width 0.3) (layer "B.Cu") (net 7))
 (segment (start 136.80543 82.008439) (end 136.8 82.003009) (width 0.3) (layer "B.Cu") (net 7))
 (segment (start 136.8 85.04) (end 136.8 82.013869) (width 0.3) (layer "B.Cu") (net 7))
 (segment (start 136.8 81.965) (end 135.6 81.965) (width 0.3) (layer "B.Cu") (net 7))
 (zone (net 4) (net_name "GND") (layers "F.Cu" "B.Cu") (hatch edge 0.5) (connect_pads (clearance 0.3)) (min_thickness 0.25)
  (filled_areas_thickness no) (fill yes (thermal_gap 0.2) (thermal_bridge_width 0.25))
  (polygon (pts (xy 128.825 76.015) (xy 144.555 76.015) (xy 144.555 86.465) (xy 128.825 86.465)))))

